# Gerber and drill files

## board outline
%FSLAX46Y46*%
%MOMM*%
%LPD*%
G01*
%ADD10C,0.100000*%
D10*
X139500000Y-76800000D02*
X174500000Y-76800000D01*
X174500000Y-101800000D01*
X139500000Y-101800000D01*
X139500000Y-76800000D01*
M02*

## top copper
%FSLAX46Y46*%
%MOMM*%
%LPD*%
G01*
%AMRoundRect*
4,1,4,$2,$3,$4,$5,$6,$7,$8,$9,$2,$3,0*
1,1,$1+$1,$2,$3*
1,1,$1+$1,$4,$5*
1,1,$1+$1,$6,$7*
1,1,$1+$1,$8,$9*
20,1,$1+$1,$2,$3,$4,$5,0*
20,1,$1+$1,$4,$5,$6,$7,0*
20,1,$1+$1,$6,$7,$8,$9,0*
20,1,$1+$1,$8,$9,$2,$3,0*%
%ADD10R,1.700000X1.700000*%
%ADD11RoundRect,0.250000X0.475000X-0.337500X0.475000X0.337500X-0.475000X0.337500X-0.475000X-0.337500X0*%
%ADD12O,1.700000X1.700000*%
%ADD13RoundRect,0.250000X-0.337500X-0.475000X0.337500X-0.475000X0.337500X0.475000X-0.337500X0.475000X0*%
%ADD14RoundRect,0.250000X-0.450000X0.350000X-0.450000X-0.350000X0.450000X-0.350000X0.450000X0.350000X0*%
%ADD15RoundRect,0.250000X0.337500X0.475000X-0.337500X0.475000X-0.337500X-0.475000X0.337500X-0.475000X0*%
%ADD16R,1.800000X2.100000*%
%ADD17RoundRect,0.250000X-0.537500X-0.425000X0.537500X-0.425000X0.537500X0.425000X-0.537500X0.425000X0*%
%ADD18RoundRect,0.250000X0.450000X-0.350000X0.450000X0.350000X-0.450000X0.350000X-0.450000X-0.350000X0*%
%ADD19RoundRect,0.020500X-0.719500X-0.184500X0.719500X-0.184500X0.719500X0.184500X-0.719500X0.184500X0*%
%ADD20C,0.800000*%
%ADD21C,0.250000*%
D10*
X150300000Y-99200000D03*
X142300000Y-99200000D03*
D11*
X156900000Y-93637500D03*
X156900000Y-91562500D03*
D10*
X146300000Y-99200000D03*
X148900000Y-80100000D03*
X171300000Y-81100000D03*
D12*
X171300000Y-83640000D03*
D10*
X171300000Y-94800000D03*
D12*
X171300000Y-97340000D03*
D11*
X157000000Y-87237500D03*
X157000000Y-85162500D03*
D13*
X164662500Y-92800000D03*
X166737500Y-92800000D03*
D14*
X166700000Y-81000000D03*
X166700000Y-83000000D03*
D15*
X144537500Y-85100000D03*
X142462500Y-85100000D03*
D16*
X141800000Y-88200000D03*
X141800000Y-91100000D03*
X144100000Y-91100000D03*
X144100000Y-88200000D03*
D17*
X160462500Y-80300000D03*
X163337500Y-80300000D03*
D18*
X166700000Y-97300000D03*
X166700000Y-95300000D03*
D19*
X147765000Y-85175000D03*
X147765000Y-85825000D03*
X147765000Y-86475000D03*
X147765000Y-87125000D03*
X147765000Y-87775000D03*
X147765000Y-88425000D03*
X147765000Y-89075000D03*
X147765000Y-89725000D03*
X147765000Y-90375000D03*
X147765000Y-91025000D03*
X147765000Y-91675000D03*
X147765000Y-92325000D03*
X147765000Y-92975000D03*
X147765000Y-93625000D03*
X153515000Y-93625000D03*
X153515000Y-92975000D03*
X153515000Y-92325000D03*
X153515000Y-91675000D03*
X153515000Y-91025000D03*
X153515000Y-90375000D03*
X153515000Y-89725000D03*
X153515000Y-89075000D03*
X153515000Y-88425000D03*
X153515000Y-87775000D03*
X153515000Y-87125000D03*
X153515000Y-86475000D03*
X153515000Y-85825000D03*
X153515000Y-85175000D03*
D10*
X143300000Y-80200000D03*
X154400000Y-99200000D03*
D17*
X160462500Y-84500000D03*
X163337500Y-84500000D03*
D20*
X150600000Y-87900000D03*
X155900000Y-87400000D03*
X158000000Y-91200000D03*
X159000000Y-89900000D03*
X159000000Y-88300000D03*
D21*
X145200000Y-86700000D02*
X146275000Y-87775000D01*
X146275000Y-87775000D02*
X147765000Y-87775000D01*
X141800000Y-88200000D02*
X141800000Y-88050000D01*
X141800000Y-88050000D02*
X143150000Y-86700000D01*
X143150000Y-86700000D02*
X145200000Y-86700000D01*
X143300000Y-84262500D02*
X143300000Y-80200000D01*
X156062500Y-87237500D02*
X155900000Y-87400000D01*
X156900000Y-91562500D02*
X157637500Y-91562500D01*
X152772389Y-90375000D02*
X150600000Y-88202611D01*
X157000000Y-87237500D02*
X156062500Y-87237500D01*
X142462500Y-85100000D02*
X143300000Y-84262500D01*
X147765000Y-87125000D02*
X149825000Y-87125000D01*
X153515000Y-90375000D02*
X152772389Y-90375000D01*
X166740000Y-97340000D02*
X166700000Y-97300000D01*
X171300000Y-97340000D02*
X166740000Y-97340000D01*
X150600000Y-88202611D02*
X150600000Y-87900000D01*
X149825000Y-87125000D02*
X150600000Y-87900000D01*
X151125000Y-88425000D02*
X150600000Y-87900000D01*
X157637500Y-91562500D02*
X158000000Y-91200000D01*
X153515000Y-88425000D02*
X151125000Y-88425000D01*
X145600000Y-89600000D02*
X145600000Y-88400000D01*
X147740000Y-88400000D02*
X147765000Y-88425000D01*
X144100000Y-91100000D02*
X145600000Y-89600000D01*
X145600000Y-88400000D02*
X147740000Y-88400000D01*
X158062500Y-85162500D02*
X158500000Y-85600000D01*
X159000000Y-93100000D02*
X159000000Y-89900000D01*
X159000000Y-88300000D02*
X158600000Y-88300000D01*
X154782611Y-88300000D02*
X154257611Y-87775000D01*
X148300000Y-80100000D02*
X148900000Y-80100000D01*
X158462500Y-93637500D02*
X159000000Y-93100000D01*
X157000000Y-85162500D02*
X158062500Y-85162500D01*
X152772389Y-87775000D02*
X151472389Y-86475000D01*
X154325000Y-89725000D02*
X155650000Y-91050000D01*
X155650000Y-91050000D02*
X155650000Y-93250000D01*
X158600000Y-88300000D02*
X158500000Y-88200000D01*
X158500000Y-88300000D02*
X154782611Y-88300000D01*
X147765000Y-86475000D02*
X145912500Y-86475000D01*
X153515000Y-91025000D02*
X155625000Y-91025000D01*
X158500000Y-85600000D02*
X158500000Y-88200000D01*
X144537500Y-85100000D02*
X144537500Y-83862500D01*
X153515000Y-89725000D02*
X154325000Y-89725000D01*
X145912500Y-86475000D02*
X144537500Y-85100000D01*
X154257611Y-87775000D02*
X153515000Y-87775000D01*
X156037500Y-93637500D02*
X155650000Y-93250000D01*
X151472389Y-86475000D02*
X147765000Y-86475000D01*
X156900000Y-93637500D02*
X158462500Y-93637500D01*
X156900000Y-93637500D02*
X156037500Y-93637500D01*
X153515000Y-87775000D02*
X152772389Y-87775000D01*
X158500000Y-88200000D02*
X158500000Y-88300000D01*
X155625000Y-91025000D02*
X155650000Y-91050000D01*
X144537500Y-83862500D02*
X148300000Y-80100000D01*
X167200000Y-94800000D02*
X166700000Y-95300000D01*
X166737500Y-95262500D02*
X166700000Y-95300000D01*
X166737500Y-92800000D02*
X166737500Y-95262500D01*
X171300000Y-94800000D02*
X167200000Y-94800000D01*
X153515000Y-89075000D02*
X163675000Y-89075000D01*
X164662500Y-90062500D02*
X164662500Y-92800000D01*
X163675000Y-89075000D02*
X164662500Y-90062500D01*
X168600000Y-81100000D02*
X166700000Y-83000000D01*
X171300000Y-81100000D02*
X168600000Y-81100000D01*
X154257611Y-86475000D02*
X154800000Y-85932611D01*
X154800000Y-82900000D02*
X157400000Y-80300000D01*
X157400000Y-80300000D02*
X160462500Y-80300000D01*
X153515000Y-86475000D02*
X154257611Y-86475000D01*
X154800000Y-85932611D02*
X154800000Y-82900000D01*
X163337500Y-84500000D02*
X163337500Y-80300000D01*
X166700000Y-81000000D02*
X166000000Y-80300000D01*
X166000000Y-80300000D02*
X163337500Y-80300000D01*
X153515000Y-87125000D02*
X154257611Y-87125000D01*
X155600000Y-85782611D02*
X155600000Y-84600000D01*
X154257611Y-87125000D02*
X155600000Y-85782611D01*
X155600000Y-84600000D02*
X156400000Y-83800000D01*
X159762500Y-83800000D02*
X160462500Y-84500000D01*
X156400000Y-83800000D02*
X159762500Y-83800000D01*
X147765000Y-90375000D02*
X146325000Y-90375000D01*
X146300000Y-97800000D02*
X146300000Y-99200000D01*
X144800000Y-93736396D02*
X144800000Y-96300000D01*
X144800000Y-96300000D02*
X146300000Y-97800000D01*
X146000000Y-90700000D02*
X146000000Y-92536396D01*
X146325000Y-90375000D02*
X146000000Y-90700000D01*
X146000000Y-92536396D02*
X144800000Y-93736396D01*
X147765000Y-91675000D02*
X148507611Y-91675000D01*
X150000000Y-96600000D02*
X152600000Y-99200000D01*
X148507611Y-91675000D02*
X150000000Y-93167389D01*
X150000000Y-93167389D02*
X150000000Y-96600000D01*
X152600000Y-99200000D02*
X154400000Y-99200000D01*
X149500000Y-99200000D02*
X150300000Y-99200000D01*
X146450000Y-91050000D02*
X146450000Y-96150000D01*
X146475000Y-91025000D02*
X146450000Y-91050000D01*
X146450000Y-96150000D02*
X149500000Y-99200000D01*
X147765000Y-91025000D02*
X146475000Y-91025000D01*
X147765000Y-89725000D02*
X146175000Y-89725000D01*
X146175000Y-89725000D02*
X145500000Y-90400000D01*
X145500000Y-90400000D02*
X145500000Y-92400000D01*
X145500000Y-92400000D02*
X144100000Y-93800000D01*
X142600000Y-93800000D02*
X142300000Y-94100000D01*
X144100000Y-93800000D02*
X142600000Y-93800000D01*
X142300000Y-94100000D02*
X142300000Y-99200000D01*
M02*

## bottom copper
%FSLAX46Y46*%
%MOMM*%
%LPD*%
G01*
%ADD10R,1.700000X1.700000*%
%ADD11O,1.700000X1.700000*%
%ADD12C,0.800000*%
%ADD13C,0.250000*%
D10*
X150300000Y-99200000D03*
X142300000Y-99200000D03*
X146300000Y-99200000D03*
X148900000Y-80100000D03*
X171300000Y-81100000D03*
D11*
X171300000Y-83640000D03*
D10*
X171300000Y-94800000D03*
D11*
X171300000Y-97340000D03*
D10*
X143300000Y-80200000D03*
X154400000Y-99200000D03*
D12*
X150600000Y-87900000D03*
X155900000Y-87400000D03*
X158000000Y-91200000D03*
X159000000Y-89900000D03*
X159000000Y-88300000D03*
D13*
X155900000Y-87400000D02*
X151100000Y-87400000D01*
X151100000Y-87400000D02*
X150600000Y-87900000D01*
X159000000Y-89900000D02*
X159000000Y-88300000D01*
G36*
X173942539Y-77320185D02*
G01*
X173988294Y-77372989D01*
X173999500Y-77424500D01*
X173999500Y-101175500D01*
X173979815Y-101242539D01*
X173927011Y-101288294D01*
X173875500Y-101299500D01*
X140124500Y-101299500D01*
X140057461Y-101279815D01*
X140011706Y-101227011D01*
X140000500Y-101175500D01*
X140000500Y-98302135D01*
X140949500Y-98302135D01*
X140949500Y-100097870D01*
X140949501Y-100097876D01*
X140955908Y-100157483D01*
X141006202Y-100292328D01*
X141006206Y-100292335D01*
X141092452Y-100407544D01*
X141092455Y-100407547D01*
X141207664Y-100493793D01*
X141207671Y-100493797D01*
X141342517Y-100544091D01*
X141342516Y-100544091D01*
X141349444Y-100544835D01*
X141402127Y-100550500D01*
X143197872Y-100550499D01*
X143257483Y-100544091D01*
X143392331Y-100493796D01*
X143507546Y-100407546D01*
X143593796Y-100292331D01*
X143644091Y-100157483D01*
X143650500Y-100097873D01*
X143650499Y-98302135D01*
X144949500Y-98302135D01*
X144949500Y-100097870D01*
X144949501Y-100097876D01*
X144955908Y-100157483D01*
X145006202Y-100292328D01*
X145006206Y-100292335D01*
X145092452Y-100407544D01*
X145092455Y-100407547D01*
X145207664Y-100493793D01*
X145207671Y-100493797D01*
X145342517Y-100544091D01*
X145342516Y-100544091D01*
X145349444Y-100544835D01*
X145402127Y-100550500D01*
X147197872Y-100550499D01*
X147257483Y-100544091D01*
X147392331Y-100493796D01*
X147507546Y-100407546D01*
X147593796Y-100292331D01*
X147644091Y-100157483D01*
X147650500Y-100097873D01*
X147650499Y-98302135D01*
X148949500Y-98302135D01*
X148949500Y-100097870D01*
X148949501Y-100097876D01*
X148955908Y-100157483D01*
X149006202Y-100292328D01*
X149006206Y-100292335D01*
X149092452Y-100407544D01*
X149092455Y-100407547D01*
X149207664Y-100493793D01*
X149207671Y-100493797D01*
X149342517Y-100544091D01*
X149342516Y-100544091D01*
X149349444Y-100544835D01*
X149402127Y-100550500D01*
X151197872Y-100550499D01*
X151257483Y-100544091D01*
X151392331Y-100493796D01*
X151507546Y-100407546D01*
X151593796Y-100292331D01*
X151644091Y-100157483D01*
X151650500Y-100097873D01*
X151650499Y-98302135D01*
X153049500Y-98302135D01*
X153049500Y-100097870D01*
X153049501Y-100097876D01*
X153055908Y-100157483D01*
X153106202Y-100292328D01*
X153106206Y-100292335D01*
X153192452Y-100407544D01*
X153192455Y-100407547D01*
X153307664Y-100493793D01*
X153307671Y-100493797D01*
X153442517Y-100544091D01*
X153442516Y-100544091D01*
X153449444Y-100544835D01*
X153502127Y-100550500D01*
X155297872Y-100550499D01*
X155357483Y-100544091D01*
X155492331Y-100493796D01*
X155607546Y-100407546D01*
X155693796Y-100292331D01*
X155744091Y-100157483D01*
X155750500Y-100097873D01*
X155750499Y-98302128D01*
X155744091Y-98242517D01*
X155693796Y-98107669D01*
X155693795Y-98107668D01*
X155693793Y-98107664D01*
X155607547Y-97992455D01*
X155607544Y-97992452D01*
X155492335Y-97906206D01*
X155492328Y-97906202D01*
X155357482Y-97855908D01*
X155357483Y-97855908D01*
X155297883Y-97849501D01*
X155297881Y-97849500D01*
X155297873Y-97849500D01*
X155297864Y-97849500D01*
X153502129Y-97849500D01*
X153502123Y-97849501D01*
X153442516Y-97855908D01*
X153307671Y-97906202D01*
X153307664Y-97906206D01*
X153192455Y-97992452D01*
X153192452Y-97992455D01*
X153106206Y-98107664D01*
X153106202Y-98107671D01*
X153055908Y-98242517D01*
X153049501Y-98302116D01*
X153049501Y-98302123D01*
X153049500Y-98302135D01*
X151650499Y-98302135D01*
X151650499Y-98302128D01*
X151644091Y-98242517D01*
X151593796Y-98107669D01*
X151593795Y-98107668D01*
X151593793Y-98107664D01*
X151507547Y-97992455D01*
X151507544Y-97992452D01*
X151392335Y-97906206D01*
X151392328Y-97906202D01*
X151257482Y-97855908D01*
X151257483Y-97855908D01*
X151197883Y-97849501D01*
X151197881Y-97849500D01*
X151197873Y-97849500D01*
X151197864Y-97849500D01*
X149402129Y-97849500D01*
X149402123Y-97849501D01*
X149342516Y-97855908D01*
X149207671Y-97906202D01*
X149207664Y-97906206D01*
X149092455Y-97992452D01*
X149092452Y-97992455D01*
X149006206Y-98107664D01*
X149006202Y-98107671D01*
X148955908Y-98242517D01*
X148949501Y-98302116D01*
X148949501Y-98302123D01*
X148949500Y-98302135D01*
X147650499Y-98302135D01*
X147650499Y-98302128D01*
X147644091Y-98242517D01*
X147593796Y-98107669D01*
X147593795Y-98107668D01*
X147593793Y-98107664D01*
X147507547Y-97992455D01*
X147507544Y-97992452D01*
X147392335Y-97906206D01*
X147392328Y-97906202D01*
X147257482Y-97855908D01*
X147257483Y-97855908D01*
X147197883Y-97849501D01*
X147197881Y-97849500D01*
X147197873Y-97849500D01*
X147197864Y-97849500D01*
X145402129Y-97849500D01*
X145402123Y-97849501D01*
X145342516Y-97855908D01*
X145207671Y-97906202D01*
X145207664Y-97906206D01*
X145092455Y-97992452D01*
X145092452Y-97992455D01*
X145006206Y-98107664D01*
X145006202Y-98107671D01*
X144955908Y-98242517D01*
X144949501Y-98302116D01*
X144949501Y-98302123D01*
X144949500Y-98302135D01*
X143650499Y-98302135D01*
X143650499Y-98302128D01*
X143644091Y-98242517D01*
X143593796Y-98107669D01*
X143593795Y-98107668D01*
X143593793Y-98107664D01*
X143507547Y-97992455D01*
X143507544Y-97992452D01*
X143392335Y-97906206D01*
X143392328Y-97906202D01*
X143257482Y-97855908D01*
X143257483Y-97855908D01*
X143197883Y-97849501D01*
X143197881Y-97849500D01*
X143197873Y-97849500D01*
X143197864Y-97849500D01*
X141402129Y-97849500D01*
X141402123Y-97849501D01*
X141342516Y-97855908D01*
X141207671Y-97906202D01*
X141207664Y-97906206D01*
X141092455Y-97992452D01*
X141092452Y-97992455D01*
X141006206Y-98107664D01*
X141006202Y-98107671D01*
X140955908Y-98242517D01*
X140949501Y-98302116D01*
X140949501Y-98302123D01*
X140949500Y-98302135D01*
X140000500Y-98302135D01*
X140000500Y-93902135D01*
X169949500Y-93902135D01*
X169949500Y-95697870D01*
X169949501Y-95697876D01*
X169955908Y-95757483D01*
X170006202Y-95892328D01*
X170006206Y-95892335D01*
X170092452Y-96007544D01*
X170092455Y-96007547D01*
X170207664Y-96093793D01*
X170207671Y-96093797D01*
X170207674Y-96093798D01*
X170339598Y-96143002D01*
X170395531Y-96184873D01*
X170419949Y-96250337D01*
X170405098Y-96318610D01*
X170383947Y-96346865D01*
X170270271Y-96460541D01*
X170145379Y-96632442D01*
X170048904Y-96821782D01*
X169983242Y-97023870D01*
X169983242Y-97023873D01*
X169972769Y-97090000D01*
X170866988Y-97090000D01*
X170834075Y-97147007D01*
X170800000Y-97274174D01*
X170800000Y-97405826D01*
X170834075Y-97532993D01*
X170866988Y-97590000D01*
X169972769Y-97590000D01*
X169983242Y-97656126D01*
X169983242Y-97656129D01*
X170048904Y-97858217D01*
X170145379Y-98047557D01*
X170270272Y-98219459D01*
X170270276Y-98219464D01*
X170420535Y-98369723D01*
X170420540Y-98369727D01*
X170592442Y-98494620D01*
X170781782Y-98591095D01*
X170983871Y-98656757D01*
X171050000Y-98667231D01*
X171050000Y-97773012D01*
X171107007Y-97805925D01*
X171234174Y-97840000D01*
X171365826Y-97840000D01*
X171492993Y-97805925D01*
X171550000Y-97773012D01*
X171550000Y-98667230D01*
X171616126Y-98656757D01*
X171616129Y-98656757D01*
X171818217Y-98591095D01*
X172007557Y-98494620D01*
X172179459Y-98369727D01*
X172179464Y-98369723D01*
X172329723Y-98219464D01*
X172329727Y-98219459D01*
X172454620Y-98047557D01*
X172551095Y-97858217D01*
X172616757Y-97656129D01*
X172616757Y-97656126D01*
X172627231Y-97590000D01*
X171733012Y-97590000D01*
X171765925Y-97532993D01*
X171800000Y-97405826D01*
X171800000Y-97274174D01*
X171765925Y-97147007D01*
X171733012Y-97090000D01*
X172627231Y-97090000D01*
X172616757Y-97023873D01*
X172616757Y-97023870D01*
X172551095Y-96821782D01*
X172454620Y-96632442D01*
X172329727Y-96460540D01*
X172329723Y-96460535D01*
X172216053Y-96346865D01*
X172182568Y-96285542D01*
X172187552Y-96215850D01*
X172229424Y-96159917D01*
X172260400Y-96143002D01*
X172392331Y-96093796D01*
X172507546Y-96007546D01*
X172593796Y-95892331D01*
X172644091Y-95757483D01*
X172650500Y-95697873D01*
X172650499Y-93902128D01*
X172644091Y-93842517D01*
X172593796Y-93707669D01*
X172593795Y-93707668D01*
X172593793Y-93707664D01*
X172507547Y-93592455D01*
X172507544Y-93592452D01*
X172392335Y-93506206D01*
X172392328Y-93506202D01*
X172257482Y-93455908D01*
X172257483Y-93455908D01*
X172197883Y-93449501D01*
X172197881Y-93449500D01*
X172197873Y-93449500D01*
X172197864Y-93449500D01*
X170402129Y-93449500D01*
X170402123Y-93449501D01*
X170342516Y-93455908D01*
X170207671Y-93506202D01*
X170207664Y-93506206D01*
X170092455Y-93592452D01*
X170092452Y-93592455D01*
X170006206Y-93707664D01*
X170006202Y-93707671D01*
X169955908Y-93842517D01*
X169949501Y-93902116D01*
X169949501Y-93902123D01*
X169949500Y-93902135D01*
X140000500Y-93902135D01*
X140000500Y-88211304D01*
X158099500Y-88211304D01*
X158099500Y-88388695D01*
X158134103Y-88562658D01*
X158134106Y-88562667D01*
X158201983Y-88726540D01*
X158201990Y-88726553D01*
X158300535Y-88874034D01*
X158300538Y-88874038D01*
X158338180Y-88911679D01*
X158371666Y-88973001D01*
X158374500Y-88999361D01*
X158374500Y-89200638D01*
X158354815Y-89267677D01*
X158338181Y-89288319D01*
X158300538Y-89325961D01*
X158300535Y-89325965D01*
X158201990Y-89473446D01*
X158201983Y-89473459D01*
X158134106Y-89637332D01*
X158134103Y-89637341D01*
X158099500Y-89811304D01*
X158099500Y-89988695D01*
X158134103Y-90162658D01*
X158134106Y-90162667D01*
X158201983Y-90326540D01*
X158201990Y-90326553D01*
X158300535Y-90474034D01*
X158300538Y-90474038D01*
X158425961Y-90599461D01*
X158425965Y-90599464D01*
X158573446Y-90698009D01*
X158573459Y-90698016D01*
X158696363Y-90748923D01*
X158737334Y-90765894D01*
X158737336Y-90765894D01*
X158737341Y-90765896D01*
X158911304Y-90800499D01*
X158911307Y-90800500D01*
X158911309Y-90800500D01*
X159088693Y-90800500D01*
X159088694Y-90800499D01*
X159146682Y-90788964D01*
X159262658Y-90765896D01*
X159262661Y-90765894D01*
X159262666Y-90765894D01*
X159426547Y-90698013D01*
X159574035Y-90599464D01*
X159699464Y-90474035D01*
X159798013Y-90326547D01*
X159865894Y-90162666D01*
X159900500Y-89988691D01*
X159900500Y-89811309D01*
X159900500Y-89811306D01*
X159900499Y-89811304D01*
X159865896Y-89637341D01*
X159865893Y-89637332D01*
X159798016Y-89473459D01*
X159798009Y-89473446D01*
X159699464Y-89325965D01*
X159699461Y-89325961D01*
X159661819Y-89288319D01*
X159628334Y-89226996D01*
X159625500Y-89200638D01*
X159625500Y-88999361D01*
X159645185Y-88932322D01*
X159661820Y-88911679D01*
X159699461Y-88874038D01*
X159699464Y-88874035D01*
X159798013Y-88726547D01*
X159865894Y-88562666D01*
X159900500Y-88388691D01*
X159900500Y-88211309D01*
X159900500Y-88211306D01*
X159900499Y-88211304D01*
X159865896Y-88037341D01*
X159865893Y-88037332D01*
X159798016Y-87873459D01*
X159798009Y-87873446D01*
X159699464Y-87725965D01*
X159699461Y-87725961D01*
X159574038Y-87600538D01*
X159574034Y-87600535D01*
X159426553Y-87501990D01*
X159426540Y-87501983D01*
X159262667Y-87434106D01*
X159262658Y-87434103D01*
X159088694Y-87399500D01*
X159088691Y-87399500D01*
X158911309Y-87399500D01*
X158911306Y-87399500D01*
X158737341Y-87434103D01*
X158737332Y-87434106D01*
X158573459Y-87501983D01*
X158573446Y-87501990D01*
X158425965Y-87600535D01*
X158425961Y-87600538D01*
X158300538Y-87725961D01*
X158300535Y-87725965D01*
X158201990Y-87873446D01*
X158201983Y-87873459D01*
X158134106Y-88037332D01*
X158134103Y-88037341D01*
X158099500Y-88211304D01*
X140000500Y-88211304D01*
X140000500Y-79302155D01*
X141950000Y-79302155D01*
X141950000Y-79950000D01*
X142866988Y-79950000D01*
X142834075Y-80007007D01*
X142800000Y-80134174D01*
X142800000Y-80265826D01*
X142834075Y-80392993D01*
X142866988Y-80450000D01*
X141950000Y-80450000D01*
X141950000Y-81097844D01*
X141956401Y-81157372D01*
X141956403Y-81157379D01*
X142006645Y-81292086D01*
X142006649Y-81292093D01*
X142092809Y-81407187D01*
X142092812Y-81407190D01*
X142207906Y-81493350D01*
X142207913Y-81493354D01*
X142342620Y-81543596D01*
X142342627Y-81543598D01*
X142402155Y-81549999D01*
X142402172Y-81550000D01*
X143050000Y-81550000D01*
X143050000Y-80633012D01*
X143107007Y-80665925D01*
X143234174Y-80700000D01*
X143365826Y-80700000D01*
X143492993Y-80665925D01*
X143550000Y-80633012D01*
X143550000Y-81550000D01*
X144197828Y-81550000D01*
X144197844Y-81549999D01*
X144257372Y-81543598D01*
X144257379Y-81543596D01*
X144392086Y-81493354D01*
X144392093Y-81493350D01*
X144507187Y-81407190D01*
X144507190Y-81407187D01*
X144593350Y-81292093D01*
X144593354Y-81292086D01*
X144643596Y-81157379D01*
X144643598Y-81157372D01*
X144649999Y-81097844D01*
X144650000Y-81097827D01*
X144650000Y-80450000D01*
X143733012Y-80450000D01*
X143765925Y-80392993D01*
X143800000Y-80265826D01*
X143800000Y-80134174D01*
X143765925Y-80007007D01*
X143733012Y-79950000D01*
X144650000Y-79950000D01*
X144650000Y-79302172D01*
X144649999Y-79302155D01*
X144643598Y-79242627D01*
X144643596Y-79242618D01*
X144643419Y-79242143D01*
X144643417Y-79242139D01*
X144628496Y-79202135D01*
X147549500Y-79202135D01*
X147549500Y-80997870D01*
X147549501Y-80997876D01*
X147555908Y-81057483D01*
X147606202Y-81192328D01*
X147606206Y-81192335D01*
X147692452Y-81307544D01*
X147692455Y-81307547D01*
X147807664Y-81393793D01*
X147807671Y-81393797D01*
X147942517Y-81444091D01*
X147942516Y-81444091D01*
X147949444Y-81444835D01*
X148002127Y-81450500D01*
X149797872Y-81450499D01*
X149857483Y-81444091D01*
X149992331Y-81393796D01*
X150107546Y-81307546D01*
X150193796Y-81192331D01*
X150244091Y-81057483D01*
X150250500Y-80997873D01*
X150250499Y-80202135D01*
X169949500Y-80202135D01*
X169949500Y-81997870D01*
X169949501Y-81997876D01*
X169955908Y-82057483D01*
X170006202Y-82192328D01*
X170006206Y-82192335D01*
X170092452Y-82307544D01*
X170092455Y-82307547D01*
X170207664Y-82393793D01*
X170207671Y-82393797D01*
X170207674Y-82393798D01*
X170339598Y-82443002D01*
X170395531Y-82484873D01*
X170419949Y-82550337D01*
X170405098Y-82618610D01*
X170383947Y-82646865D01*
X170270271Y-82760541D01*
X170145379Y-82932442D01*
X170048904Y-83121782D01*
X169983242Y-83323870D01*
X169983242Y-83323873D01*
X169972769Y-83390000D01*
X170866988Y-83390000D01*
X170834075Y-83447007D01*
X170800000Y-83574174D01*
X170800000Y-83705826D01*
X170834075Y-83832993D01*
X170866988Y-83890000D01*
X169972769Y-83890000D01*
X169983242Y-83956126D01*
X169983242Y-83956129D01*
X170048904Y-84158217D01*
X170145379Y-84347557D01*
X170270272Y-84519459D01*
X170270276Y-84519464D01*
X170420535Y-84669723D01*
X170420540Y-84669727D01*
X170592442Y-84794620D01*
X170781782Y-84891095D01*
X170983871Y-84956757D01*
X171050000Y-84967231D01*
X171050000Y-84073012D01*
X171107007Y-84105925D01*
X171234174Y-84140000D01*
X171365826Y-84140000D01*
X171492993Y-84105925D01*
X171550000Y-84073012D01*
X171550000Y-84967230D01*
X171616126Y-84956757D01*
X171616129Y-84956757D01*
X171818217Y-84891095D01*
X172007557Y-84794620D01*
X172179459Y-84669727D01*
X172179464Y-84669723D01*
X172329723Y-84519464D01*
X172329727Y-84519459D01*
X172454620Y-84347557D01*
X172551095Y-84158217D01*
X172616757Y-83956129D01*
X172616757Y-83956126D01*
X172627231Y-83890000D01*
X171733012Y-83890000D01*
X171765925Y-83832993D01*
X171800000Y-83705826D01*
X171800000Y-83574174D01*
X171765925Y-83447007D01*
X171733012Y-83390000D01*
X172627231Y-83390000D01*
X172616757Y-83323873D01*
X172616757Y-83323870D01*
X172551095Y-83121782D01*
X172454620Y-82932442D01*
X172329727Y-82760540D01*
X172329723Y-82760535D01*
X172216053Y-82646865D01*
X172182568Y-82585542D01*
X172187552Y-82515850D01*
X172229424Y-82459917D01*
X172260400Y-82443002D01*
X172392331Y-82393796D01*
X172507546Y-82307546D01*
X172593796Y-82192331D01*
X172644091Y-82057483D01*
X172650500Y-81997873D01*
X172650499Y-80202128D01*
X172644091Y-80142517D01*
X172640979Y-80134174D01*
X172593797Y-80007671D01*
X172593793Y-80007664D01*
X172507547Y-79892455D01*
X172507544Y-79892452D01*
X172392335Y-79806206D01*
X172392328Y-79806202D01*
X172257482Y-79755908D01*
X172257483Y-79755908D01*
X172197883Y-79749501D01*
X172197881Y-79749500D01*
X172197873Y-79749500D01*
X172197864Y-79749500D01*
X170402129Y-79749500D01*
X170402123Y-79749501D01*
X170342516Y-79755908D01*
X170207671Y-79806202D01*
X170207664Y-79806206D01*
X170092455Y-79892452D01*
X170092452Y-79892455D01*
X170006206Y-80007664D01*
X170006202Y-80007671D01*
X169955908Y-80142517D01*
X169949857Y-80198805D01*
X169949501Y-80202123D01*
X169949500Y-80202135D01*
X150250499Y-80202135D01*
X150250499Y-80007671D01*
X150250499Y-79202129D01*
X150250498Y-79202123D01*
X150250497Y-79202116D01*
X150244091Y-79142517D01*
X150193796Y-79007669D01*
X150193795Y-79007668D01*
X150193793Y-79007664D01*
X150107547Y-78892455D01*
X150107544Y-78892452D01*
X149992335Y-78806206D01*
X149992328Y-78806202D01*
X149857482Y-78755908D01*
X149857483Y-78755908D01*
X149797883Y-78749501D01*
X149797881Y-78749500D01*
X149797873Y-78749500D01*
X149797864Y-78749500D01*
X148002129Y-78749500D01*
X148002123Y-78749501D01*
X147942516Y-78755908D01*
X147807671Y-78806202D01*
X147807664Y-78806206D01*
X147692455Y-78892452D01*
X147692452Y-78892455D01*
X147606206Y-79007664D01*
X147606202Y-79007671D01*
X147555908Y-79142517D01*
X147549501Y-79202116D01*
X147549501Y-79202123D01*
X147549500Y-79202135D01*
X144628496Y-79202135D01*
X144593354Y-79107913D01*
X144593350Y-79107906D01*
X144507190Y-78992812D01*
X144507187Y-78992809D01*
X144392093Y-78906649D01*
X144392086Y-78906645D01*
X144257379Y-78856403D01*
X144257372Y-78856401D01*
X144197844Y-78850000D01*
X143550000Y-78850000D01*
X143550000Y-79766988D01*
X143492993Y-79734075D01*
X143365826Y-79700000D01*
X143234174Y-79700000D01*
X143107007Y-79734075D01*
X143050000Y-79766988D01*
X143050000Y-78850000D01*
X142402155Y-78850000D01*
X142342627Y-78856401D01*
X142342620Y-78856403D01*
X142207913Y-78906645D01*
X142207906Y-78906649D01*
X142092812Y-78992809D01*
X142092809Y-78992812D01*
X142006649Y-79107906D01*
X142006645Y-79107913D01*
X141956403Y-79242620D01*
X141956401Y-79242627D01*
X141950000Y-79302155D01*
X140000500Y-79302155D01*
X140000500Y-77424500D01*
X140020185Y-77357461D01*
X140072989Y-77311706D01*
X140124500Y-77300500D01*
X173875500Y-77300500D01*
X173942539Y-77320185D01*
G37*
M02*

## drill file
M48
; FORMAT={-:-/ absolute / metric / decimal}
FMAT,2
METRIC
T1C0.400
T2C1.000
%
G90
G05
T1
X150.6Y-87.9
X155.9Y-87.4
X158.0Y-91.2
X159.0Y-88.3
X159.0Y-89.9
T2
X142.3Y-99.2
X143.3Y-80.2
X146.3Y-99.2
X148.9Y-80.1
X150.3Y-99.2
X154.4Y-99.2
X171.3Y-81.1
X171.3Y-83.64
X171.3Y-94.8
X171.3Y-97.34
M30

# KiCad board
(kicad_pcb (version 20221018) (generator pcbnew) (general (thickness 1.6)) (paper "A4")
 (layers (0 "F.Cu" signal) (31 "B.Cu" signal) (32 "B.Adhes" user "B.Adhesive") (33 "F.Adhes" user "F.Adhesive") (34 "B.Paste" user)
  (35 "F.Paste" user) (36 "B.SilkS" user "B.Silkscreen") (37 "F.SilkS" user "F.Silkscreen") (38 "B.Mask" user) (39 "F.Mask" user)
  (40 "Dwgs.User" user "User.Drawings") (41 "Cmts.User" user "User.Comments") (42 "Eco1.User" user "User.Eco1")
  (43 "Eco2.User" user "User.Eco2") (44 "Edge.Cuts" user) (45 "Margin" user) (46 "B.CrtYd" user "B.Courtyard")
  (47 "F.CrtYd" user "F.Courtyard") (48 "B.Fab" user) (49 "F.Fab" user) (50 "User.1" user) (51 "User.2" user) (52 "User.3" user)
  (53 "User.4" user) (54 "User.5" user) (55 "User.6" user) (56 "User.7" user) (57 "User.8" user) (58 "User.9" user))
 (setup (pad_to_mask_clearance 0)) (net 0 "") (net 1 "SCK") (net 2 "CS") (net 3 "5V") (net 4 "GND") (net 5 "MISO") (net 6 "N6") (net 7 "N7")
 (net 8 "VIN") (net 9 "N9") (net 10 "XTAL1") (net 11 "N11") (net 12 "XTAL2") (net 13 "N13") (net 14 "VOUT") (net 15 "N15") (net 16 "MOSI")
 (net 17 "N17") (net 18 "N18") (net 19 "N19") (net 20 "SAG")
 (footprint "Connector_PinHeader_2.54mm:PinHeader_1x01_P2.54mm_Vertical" (layer "F.Cu") (at 150.3 99.2)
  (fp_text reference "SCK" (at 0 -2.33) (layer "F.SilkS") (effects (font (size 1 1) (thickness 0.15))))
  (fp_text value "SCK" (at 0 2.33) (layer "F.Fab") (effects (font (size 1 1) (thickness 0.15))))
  (pad "1" thru_hole rect (at 0 0) (size 1.7 1.7) (drill 1) (layers "*.Cu" "*.Mask") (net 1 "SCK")))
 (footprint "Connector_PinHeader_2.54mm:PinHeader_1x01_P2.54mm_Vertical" (layer "F.Cu") (at 142.3 99.2)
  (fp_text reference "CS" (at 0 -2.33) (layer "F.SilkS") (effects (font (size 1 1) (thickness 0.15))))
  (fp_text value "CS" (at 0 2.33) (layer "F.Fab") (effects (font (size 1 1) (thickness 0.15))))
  (pad "1" thru_hole rect (at 0 0) (size 1.7 1.7) (drill 1) (layers "*.Cu" "*.Mask") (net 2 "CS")))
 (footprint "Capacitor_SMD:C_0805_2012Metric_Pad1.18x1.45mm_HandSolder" (layer "F.Cu") (at 156.9 92.6 90)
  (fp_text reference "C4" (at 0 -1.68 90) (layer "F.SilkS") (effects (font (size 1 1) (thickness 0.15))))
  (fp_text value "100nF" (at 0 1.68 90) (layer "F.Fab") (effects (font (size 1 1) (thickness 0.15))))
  (pad "1" smd roundrect (at -1.0375 0 90) (size 1.175 1.45) (layers "F.Cu" "F.Paste" "F.Mask") (roundrect_rratio 0.212766) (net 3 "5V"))
  (pad "2" smd roundrect (at 1.0375 0 90) (size 1.175 1.45) (layers "F.Cu" "F.Paste" "F.Mask") (roundrect_rratio 0.212766) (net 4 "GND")))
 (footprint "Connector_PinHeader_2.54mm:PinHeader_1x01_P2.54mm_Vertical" (layer "F.Cu") (at 146.3 99.2)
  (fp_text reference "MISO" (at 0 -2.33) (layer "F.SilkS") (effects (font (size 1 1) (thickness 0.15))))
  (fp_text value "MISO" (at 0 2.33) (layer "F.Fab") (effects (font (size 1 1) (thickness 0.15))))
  (pad "1" thru_hole rect (at 0 0) (size 1.7 1.7) (drill 1) (layers "*.Cu" "*.Mask") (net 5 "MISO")))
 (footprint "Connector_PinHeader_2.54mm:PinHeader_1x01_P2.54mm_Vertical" (layer "F.Cu") (at 148.9 80.1)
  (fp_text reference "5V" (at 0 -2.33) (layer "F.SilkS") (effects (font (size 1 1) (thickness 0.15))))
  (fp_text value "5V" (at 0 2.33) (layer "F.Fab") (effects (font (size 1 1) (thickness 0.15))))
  (pad "1" thru_hole rect (at 0 0) (size 1.7 1.7) (drill 1) (layers "*.Cu" "*.Mask") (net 3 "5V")))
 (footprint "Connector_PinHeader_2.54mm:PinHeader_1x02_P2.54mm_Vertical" (layer "F.Cu") (at 171.3 81.1)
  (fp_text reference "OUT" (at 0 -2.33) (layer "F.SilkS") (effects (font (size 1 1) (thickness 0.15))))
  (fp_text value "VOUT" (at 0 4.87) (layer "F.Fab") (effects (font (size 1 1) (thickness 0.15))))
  (pad "1" thru_hole rect (at 0 0) (size 1.7 1.7) (drill 1) (layers "*.Cu" "*.Mask") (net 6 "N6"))
  (pad "2" thru_hole oval (at 0 2.54) (size 1.7 1.7) (drill 1) (layers "*.Cu" "*.Mask") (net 4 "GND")))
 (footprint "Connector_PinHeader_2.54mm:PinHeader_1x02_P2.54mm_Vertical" (layer "F.Cu") (at 171.3 94.8)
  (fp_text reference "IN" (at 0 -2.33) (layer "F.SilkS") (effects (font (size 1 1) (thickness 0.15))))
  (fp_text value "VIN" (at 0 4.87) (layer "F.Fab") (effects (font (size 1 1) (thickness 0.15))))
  (pad "1" thru_hole rect (at 0 0) (size 1.7 1.7) (drill 1) (layers "*.Cu" "*.Mask") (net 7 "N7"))
  (pad "2" thru_hole oval (at 0 2.54) (size 1.7 1.7) (drill 1) (layers "*.Cu" "*.Mask") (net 4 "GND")))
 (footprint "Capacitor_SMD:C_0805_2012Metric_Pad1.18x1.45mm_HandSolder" (layer "F.Cu") (at 157 86.2 90)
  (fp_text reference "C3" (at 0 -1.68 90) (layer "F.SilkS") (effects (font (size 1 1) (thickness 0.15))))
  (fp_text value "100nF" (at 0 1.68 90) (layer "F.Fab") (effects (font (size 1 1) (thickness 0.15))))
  (pad "1" smd roundrect (at -1.0375 0 90) (size 1.175 1.45) (layers "F.Cu" "F.Paste" "F.Mask") (roundrect_rratio 0.212766) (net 4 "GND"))
  (pad "2" smd roundrect (at 1.0375 0 90) (size 1.175 1.45) (layers "F.Cu" "F.Paste" "F.Mask") (roundrect_rratio 0.212766) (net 3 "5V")))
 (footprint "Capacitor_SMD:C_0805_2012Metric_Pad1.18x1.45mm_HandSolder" (layer "F.Cu") (at 165.7 92.8)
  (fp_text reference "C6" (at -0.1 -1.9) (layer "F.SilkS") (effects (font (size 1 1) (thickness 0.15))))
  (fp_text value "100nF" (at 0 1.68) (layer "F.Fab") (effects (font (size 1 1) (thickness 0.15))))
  (pad "1" smd roundrect (at -1.0375 0) (size 1.175 1.45) (layers "F.Cu" "F.Paste" "F.Mask") (roundrect_rratio 0.212766) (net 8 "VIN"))
  (pad "2" smd roundrect (at 1.0375 0) (size 1.175 1.45) (layers "F.Cu" "F.Paste" "F.Mask") (roundrect_rratio 0.212766) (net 7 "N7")))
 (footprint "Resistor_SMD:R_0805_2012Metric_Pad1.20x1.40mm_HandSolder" (layer "F.Cu") (at 166.7 82 -90)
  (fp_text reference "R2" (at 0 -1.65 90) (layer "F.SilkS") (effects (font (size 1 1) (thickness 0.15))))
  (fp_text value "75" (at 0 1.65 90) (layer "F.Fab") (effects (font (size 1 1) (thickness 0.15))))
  (pad "1" smd roundrect (at -1 0 270) (size 1.2 1.4) (layers "F.Cu" "F.Paste" "F.Mask") (roundrect_rratio 0.208333) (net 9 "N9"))
  (pad "2" smd roundrect (at 1 0 270) (size 1.2 1.4) (layers "F.Cu" "F.Paste" "F.Mask") (roundrect_rratio 0.208333) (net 6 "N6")))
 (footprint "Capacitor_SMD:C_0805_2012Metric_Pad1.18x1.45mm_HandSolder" (layer "F.Cu") (at 143.5 85.1 180)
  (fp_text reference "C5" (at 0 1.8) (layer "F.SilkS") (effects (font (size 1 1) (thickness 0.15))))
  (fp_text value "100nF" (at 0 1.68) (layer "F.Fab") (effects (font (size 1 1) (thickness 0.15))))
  (pad "1" smd roundrect (at -1.0375 0 180) (size 1.175 1.45) (layers "F.Cu" "F.Paste" "F.Mask") (roundrect_rratio 0.212766) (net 3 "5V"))
  (pad "2" smd roundrect (at 1.0375 0 180) (size 1.175 1.45) (layers "F.Cu" "F.Paste" "F.Mask") (roundrect_rratio 0.212766) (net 4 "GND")))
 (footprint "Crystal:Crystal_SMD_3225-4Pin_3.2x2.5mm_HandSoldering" (layer "F.Cu") (at 142.95 89.65 -90)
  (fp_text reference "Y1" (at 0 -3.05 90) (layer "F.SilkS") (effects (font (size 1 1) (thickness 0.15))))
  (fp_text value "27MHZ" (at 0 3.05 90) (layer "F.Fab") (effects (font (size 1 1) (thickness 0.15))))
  (pad "1" smd rect (at -1.45 1.15 270) (size 2.1 1.8) (layers "F.Cu" "F.Paste" "F.Mask") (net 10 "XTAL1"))
  (pad "2" smd rect (at 1.45 1.15 270) (size 2.1 1.8) (layers "F.Cu" "F.Paste" "F.Mask") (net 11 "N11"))
  (pad "3" smd rect (at 1.45 -1.15 270) (size 2.1 1.8) (layers "F.Cu" "F.Paste" "F.Mask") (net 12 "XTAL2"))
  (pad "4" smd rect (at -1.45 -1.15 270) (size 2.1 1.8) (layers "F.Cu" "F.Paste" "F.Mask") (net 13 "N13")))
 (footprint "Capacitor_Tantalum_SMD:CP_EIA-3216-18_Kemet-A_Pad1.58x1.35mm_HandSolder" (layer "F.Cu") (at 161.9 80.3)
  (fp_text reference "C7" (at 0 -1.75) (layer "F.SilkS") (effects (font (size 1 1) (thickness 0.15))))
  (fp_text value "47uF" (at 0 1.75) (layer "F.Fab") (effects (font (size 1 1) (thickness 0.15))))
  (pad "1" smd roundrect (at -1.4375 0) (size 1.575 1.35) (layers "F.Cu" "F.Paste" "F.Mask") (roundrect_rratio 0.185185) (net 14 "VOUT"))
  (pad "2" smd roundrect (at 1.4375 0) (size 1.575 1.35) (layers "F.Cu" "F.Paste" "F.Mask") (roundrect_rratio 0.185185) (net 9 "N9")))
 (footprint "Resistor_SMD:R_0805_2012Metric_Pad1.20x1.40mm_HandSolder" (layer "F.Cu") (at 166.7 96.3 90)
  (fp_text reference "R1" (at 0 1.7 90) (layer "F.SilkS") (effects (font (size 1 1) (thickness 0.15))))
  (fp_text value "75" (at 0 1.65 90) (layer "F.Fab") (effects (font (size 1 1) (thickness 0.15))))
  (pad "1" smd roundrect (at -1 0 90) (size 1.2 1.4) (layers "F.Cu" "F.Paste" "F.Mask") (roundrect_rratio 0.208333) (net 4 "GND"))
  (pad "2" smd roundrect (at 1 0 90) (size 1.2 1.4) (layers "F.Cu" "F.Paste" "F.Mask") (roundrect_rratio 0.208333) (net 7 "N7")))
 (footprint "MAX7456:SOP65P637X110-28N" (layer "F.Cu") (at 150.64 89.4)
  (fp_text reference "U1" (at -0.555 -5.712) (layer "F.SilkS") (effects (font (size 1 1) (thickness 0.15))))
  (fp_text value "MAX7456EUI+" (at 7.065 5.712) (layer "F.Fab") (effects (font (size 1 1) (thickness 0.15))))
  (pad "1" smd roundrect (at -2.875 -4.225) (size 1.48 0.41) (layers "F.Cu" "F.Paste" "F.Mask") (roundrect_rratio 0.05))
  (pad "2" smd roundrect (at -2.875 -3.575) (size 1.48 0.41) (layers "F.Cu" "F.Paste" "F.Mask") (roundrect_rratio 0.05))
  (pad "3" smd roundrect (at -2.875 -2.925) (size 1.48 0.41) (layers "F.Cu" "F.Paste" "F.Mask") (roundrect_rratio 0.05) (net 3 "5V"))
  (pad "4" smd roundrect (at -2.875 -2.275) (size 1.48 0.41) (layers "F.Cu" "F.Paste" "F.Mask") (roundrect_rratio 0.05) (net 4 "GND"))
  (pad "5" smd roundrect (at -2.875 -1.625) (size 1.48 0.41) (layers "F.Cu" "F.Paste" "F.Mask") (roundrect_rratio 0.05) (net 10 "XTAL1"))
  (pad "6" smd roundrect (at -2.875 -0.975) (size 1.48 0.41) (layers "F.Cu" "F.Paste" "F.Mask") (roundrect_rratio 0.05) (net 12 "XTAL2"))
  (pad "7" smd roundrect (at -2.875 -0.325) (size 1.48 0.41) (layers "F.Cu" "F.Paste" "F.Mask") (roundrect_rratio 0.05) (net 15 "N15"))
  (pad "8" smd roundrect (at -2.875 0.325) (size 1.48 0.41) (layers "F.Cu" "F.Paste" "F.Mask") (roundrect_rratio 0.05) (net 2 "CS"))
  (pad "9" smd roundrect (at -2.875 0.975) (size 1.48 0.41) (layers "F.Cu" "F.Paste" "F.Mask") (roundrect_rratio 0.05) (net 5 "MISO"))
  (pad "10" smd roundrect (at -2.875 1.625) (size 1.48 0.41) (layers "F.Cu" "F.Paste" "F.Mask") (roundrect_rratio 0.05) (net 1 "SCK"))
  (pad "11" smd roundrect (at -2.875 2.275) (size 1.48 0.41) (layers "F.Cu" "F.Paste" "F.Mask") (roundrect_rratio 0.05) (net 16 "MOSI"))
  (pad "12" smd roundrect (at -2.875 2.925) (size 1.48 0.41) (layers "F.Cu" "F.Paste" "F.Mask") (roundrect_rratio 0.05) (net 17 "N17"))
  (pad "13" smd roundrect (at -2.875 3.575) (size 1.48 0.41) (layers "F.Cu" "F.Paste" "F.Mask") (roundrect_rratio 0.05))
  (pad "14" smd roundrect (at -2.875 4.225) (size 1.48 0.41) (layers "F.Cu" "F.Paste" "F.Mask") (roundrect_rratio 0.05))
  (pad "15" smd roundrect (at 2.875 4.225) (size 1.48 0.41) (layers "F.Cu" "F.Paste" "F.Mask") (roundrect_rratio 0.05))
  (pad "16" smd roundrect (at 2.875 3.575) (size 1.48 0.41) (layers "F.Cu" "F.Paste" "F.Mask") (roundrect_rratio 0.05))
  (pad "17" smd roundrect (at 2.875 2.925) (size 1.48 0.41) (layers "F.Cu" "F.Paste" "F.Mask") (roundrect_rratio 0.05) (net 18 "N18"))
  (pad "18" smd roundrect (at 2.875 2.275) (size 1.48 0.41) (layers "F.Cu" "F.Paste" "F.Mask") (roundrect_rratio 0.05) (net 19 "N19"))
  (pad "19" smd roundrect (at 2.875 1.625) (size 1.48 0.41) (layers "F.Cu" "F.Paste" "F.Mask") (roundrect_rratio 0.05) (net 3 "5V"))
  (pad "20" smd roundrect (at 2.875 0.975) (size 1.48 0.41) (layers "F.Cu" "F.Paste" "F.Mask") (roundrect_rratio 0.05) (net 4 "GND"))
  (pad "21" smd roundrect (at 2.875 0.325) (size 1.48 0.41) (layers "F.Cu" "F.Paste" "F.Mask") (roundrect_rratio 0.05) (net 3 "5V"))
  (pad "22" smd roundrect (at 2.875 -0.325) (size 1.48 0.41) (layers "F.Cu" "F.Paste" "F.Mask") (roundrect_rratio 0.05) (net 8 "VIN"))
  (pad "23" smd roundrect (at 2.875 -0.975) (size 1.48 0.41) (layers "F.Cu" "F.Paste" "F.Mask") (roundrect_rratio 0.05) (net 4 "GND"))
  (pad "24" smd roundrect (at 2.875 -1.625) (size 1.48 0.41) (layers "F.Cu" "F.Paste" "F.Mask") (roundrect_rratio 0.05) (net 3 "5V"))
  (pad "25" smd roundrect (at 2.875 -2.275) (size 1.48 0.41) (layers "F.Cu" "F.Paste" "F.Mask") (roundrect_rratio 0.05) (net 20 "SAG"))
  (pad "26" smd roundrect (at 2.875 -2.925) (size 1.48 0.41) (layers "F.Cu" "F.Paste" "F.Mask") (roundrect_rratio 0.05) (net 14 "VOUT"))
  (pad "27" smd roundrect (at 2.875 -3.575) (size 1.48 0.41) (layers "F.Cu" "F.Paste" "F.Mask") (roundrect_rratio 0.05))
  (pad "28" smd roundrect (at 2.875 -4.225) (size 1.48 0.41) (layers "F.Cu" "F.Paste" "F.Mask") (roundrect_rratio 0.05)))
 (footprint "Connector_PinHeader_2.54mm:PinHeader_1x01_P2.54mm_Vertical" (layer "F.Cu") (at 143.3 80.2)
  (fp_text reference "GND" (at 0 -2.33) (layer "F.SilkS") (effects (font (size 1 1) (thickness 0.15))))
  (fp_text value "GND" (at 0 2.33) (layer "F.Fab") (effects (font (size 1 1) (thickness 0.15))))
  (pad "1" thru_hole rect (at 0 0) (size 1.7 1.7) (drill 1) (layers "*.Cu" "*.Mask") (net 4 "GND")))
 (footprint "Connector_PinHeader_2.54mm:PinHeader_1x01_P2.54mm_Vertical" (layer "F.Cu") (at 154.4 99.2)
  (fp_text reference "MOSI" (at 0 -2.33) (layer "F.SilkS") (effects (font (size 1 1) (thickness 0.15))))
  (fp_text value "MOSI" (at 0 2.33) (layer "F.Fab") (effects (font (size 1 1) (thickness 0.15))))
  (pad "1" thru_hole rect (at 0 0) (size 1.7 1.7) (drill 1) (layers "*.Cu" "*.Mask") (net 16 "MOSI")))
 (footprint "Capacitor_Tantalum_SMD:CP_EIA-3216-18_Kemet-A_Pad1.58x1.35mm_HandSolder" (layer "F.Cu") (at 161.9 84.5)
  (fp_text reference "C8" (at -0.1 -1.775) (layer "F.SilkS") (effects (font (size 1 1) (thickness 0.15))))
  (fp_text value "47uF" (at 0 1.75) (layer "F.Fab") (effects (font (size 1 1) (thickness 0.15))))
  (pad "1" smd roundrect (at -1.4375 0) (size 1.575 1.35) (layers "F.Cu" "F.Paste" "F.Mask") (roundrect_rratio 0.185185) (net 20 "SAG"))
  (pad "2" smd roundrect (at 1.4375 0) (size 1.575 1.35) (layers "F.Cu" "F.Paste" "F.Mask") (roundrect_rratio 0.185185) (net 9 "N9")))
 (gr_rect (start 139.5 76.8) (end 174.5 101.8) (stroke (width 0.1) (type default)) (fill none) (layer "Edge.Cuts"))
 (segment (start 145.2 86.7) (end 146.275 87.775) (width 0.25) (layer "F.Cu") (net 10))
 (segment (start 146.275 87.775) (end 147.765 87.775) (width 0.25) (layer "F.Cu") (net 10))
 (segment (start 141.8 88.2) (end 141.8 88.05) (width 0.25) (layer "F.Cu") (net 10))
 (segment (start 141.8 88.05) (end 143.15 86.7) (width 0.25) (layer "F.Cu") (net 10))
 (segment (start 143.15 86.7) (end 145.2 86.7) (width 0.25) (layer "F.Cu") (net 10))
 (segment (start 143.3 84.2625) (end 143.3 80.2) (width 0.25) (layer "F.Cu") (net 4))
 (segment (start 156.0625 87.2375) (end 155.9 87.4) (width 0.25) (layer "F.Cu") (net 4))
 (segment (start 156.9 91.5625) (end 157.6375 91.5625) (width 0.25) (layer "F.Cu") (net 4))
 (segment (start 152.772389 90.375) (end 150.6 88.202611) (width 0.25) (layer "F.Cu") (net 4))
 (segment (start 157 87.2375) (end 156.0625 87.2375) (width 0.25) (layer "F.Cu") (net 4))
 (segment (start 142.4625 85.1) (end 143.3 84.2625) (width 0.25) (layer "F.Cu") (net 4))
 (segment (start 147.765 87.125) (end 149.825 87.125) (width 0.25) (layer "F.Cu") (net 4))
 (segment (start 153.515 90.375) (end 152.772389 90.375) (width 0.25) (layer "F.Cu") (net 4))
 (segment (start 166.74 97.34) (end 166.7 97.3) (width 0.25) (layer "F.Cu") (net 4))
 (segment (start 171.3 97.34) (end 166.74 97.34) (width 0.25) (layer "F.Cu") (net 4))
 (segment (start 150.6 88.202611) (end 150.6 87.9) (width 0.25) (layer "F.Cu") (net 4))
 (segment (start 149.825 87.125) (end 150.6 87.9) (width 0.25) (layer "F.Cu") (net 4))
 (segment (start 151.125 88.425) (end 150.6 87.9) (width 0.25) (layer "F.Cu") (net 4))
 (segment (start 157.6375 91.5625) (end 158 91.2) (width 0.25) (layer "F.Cu") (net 4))
 (segment (start 153.515 88.425) (end 151.125 88.425) (width 0.25) (layer "F.Cu") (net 4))
 (via (at 150.6 87.9) (size 0.8) (drill 0.4) (layers "F.Cu" "B.Cu") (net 4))
 (via (at 155.9 87.4) (size 0.8) (drill 0.4) (layers "F.Cu" "B.Cu") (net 4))
 (via (at 158 91.2) (size 0.8) (drill 0.4) (layers "F.Cu" "B.Cu") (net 4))
 (segment (start 155.9 87.4) (end 151.1 87.4) (width 0.25) (layer "B.Cu") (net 4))
 (segment (start 151.1 87.4) (end 150.6 87.9) (width 0.25) (layer "B.Cu") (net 4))
 (segment (start 145.6 89.6) (end 145.6 88.4) (width 0.25) (layer "F.Cu") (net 12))
 (segment (start 147.74 88.4) (end 147.765 88.425) (width 0.25) (layer "F.Cu") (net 12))
 (segment (start 144.1 91.1) (end 145.6 89.6) (width 0.25) (layer "F.Cu") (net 12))
 (segment (start 145.6 88.4) (end 147.74 88.4) (width 0.25) (layer "F.Cu") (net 12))
 (segment (start 158.0625 85.1625) (end 158.5 85.6) (width 0.25) (layer "F.Cu") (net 3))
 (segment (start 159 93.1) (end 159 89.9) (width 0.25) (layer "F.Cu") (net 3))
 (segment (start 159 88.3) (end 158.6 88.3) (width 0.25) (layer "F.Cu") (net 3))
 (segment (start 154.782611 88.3) (end 154.257611 87.775) (width 0.25) (layer "F.Cu") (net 3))
 (segment (start 148.3 80.1) (end 148.9 80.1) (width 0.25) (layer "F.Cu") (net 3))
 (segment (start 158.4625 93.6375) (end 159 93.1) (width 0.25) (layer "F.Cu") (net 3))
 (segment (start 157 85.1625) (end 158.0625 85.1625) (width 0.25) (layer "F.Cu") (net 3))
 (segment (start 152.772389 87.775) (end 151.472389 86.475) (width 0.25) (layer "F.Cu") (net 3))
 (segment (start 154.325 89.725) (end 155.65 91.05) (width 0.25) (layer "F.Cu") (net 3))
 (segment (start 155.65 91.05) (end 155.65 93.25) (width 0.25) (layer "F.Cu") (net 3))
 (segment (start 158.6 88.3) (end 158.5 88.2) (width 0.25) (layer "F.Cu") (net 3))
 (segment (start 158.5 88.3) (end 154.782611 88.3) (width 0.25) (layer "F.Cu") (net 3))
 (segment (start 147.765 86.475) (end 145.9125 86.475) (width 0.25) (layer "F.Cu") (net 3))
 (segment (start 153.515 91.025) (end 155.625 91.025) (width 0.25) (layer "F.Cu") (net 3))
 (segment (start 158.5 85.6) (end 158.5 88.2) (width 0.25) (layer "F.Cu") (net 3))
 (segment (start 144.5375 85.1) (end 144.5375 83.8625) (width 0.25) (layer "F.Cu") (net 3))
 (segment (start 153.515 89.725) (end 154.325 89.725) (width 0.25) (layer "F.Cu") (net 3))
 (segment (start 145.9125 86.475) (end 144.5375 85.1) (width 0.25) (layer "F.Cu") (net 3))
 (segment (start 154.257611 87.775) (end 153.515 87.775) (width 0.25) (layer "F.Cu") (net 3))
 (segment (start 156.0375 93.6375) (end 155.65 93.25) (width 0.25) (layer "F.Cu") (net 3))
 (segment (start 151.472389 86.475) (end 147.765 86.475) (width 0.25) (layer "F.Cu") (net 3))
 (segment (start 156.9 93.6375) (end 158.4625 93.6375) (width 0.25) (layer "F.Cu") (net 3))
 (segment (start 156.9 93.6375) (end 156.0375 93.6375) (width 0.25) (layer "F.Cu") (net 3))
 (segment (start 153.515 87.775) (end 152.772389 87.775) (width 0.25) (layer "F.Cu") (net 3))
 (segment (start 158.5 88.2) (end 158.5 88.3) (width 0.25) (layer "F.Cu") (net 3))
 (segment (start 155.625 91.025) (end 155.65 91.05) (width 0.25) (layer "F.Cu") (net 3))
 (segment (start 144.5375 83.8625) (end 148.3 80.1) (width 0.25) (layer "F.Cu") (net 3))
 (via (at 159 89.9) (size 0.8) (drill 0.4) (layers "F.Cu" "B.Cu") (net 3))
 (via (at 159 88.3) (size 0.8) (drill 0.4) (layers "F.Cu" "B.Cu") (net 3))
 (segment (start 159 89.9) (end 159 88.3) (width 0.25) (layer "B.Cu") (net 3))
 (segment (start 167.2 94.8) (end 166.7 95.3) (width 0.25) (layer "F.Cu") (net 7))
 (segment (start 166.7375 95.2625) (end 166.7 95.3) (width 0.25) (layer "F.Cu") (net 7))
 (segment (start 166.7375 92.8) (end 166.7375 95.2625) (width 0.25) (layer "F.Cu") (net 7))
 (segment (start 171.3 94.8) (end 167.2 94.8) (width 0.25) (layer "F.Cu") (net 7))
 (segment (start 153.515 89.075) (end 163.675 89.075) (width 0.25) (layer "F.Cu") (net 8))
 (segment (start 164.6625 90.0625) (end 164.6625 92.8) (width 0.25) (layer "F.Cu") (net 8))
 (segment (start 163.675 89.075) (end 164.6625 90.0625) (width 0.25) (layer "F.Cu") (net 8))
 (segment (start 168.6 81.1) (end 166.7 83) (width 0.25) (layer "F.Cu") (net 6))
 (segment (start 171.3 81.1) (end 168.6 81.1) (width 0.25) (layer "F.Cu") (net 6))
 (segment (start 154.257611 86.475) (end 154.8 85.932611) (width 0.25) (layer "F.Cu") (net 14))
 (segment (start 154.8 82.9) (end 157.4 80.3) (width 0.25) (layer "F.Cu") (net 14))
 (segment (start 157.4 80.3) (end 160.4625 80.3) (width 0.25) (layer "F.Cu") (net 14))
 (segment (start 153.515 86.475) (end 154.257611 86.475) (width 0.25) (layer "F.Cu") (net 14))
 (segment (start 154.8 85.932611) (end 154.8 82.9) (width 0.25) (layer "F.Cu") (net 14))
 (segment (start 163.3375 84.5) (end 163.3375 80.3) (width 0.25) (layer "F.Cu") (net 9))
 (segment (start 166.7 81) (end 166 80.3) (width 0.25) (layer "F.Cu") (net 9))
 (segment (start 166 80.3) (end 163.3375 80.3) (width 0.25) (layer "F.Cu") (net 9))
 (segment (start 153.515 87.125) (end 154.257611 87.125) (width 0.25) (layer "F.Cu") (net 20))
 (segment (start 155.6 85.782611) (end 155.6 84.6) (width 0.25) (layer "F.Cu") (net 20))
 (segment (start 154.257611 87.125) (end 155.6 85.782611) (width 0.25) (layer "F.Cu") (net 20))
 (segment (start 155.6 84.6) (end 156.4 83.8) (width 0.25) (layer "F.Cu") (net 20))
 (segment (start 159.7625 83.8) (end 160.4625 84.5) (width 0.25) (layer "F.Cu") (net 20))
 (segment (start 156.4 83.8) (end 159.7625 83.8) (width 0.25) (layer "F.Cu") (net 20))
 (segment (start 147.765 90.375) (end 146.325 90.375) (width 0.25) (layer "F.Cu") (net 5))
 (segment (start 146.3 97.8) (end 146.3 99.2) (width 0.25) (layer "F.Cu") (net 5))
 (segment (start 144.8 93.736396) (end 144.8 96.3) (width 0.25) (layer "F.Cu") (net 5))
 (segment (start 144.8 96.3) (end 146.3 97.8) (width 0.25) (layer "F.Cu") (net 5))
 (segment (start 146 90.7) (end 146 92.536396) (width 0.25) (layer "F.Cu") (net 5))
 (segment (start 146.325 90.375) (end 146 90.7) (width 0.25) (layer "F.Cu") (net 5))
 (segment (start 146 92.536396) (end 144.8 93.736396) (width 0.25) (layer "F.Cu") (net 5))
 (segment (start 147.765 91.675) (end 148.507611 91.675) (width 0.25) (layer "F.Cu") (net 16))
 (segment (start 150 96.6) (end 152.6 99.2) (width 0.25) (layer "F.Cu") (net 16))
 (segment (start 148.507611 91.675) (end 150 93.167389) (width 0.25) (layer "F.Cu") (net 16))
 (segment (start 150 93.167389) (end 150 96.6) (width 0.25) (layer "F.Cu") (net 16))
 (segment (start 152.6 99.2) (end 154.4 99.2) (width 0.25) (layer "F.Cu") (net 16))
 (segment (start 149.5 99.2) (end 150.3 99.2) (width 0.25) (layer "F.Cu") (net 1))
 (segment (start 146.45 91.05) (end 146.45 96.15) (width 0.25) (layer "F.Cu") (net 1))
 (segment (start 146.475 91.025) (end 146.45 91.05) (width 0.25) (layer "F.Cu") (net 1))
 (segment (start 146.45 96.15) (end 149.5 99.2) (width 0.25) (layer "F.Cu") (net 1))
 (segment (start 147.765 91.025) (end 146.475 91.025) (width 0.25) (layer "F.Cu") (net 1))
 (segment (start 147.765 89.725) (end 146.175 89.725) (width 0.25) (layer "F.Cu") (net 2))
 (segment (start 146.175 89.725) (end 145.5 90.4) (width 0.25) (layer "F.Cu") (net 2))
 (segment (start 145.5 90.4) (end 145.5 92.4) (width 0.25) (layer "F.Cu") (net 2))
 (segment (start 145.5 92.4) (end 144.1 93.8) (width 0.25) (layer "F.Cu") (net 2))
 (segment (start 142.6 93.8) (end 142.3 94.1) (width 0.25) (layer "F.Cu") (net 2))
 (segment (start 144.1 93.8) (end 142.6 93.8) (width 0.25) (layer "F.Cu") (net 2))
 (segment (start 142.3 94.1) (end 142.3 99.2) (width 0.25) (layer "F.Cu") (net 2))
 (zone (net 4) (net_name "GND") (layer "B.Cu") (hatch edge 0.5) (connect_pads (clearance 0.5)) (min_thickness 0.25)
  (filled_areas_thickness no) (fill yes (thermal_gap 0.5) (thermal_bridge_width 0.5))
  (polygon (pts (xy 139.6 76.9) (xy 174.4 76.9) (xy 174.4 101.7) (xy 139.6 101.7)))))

